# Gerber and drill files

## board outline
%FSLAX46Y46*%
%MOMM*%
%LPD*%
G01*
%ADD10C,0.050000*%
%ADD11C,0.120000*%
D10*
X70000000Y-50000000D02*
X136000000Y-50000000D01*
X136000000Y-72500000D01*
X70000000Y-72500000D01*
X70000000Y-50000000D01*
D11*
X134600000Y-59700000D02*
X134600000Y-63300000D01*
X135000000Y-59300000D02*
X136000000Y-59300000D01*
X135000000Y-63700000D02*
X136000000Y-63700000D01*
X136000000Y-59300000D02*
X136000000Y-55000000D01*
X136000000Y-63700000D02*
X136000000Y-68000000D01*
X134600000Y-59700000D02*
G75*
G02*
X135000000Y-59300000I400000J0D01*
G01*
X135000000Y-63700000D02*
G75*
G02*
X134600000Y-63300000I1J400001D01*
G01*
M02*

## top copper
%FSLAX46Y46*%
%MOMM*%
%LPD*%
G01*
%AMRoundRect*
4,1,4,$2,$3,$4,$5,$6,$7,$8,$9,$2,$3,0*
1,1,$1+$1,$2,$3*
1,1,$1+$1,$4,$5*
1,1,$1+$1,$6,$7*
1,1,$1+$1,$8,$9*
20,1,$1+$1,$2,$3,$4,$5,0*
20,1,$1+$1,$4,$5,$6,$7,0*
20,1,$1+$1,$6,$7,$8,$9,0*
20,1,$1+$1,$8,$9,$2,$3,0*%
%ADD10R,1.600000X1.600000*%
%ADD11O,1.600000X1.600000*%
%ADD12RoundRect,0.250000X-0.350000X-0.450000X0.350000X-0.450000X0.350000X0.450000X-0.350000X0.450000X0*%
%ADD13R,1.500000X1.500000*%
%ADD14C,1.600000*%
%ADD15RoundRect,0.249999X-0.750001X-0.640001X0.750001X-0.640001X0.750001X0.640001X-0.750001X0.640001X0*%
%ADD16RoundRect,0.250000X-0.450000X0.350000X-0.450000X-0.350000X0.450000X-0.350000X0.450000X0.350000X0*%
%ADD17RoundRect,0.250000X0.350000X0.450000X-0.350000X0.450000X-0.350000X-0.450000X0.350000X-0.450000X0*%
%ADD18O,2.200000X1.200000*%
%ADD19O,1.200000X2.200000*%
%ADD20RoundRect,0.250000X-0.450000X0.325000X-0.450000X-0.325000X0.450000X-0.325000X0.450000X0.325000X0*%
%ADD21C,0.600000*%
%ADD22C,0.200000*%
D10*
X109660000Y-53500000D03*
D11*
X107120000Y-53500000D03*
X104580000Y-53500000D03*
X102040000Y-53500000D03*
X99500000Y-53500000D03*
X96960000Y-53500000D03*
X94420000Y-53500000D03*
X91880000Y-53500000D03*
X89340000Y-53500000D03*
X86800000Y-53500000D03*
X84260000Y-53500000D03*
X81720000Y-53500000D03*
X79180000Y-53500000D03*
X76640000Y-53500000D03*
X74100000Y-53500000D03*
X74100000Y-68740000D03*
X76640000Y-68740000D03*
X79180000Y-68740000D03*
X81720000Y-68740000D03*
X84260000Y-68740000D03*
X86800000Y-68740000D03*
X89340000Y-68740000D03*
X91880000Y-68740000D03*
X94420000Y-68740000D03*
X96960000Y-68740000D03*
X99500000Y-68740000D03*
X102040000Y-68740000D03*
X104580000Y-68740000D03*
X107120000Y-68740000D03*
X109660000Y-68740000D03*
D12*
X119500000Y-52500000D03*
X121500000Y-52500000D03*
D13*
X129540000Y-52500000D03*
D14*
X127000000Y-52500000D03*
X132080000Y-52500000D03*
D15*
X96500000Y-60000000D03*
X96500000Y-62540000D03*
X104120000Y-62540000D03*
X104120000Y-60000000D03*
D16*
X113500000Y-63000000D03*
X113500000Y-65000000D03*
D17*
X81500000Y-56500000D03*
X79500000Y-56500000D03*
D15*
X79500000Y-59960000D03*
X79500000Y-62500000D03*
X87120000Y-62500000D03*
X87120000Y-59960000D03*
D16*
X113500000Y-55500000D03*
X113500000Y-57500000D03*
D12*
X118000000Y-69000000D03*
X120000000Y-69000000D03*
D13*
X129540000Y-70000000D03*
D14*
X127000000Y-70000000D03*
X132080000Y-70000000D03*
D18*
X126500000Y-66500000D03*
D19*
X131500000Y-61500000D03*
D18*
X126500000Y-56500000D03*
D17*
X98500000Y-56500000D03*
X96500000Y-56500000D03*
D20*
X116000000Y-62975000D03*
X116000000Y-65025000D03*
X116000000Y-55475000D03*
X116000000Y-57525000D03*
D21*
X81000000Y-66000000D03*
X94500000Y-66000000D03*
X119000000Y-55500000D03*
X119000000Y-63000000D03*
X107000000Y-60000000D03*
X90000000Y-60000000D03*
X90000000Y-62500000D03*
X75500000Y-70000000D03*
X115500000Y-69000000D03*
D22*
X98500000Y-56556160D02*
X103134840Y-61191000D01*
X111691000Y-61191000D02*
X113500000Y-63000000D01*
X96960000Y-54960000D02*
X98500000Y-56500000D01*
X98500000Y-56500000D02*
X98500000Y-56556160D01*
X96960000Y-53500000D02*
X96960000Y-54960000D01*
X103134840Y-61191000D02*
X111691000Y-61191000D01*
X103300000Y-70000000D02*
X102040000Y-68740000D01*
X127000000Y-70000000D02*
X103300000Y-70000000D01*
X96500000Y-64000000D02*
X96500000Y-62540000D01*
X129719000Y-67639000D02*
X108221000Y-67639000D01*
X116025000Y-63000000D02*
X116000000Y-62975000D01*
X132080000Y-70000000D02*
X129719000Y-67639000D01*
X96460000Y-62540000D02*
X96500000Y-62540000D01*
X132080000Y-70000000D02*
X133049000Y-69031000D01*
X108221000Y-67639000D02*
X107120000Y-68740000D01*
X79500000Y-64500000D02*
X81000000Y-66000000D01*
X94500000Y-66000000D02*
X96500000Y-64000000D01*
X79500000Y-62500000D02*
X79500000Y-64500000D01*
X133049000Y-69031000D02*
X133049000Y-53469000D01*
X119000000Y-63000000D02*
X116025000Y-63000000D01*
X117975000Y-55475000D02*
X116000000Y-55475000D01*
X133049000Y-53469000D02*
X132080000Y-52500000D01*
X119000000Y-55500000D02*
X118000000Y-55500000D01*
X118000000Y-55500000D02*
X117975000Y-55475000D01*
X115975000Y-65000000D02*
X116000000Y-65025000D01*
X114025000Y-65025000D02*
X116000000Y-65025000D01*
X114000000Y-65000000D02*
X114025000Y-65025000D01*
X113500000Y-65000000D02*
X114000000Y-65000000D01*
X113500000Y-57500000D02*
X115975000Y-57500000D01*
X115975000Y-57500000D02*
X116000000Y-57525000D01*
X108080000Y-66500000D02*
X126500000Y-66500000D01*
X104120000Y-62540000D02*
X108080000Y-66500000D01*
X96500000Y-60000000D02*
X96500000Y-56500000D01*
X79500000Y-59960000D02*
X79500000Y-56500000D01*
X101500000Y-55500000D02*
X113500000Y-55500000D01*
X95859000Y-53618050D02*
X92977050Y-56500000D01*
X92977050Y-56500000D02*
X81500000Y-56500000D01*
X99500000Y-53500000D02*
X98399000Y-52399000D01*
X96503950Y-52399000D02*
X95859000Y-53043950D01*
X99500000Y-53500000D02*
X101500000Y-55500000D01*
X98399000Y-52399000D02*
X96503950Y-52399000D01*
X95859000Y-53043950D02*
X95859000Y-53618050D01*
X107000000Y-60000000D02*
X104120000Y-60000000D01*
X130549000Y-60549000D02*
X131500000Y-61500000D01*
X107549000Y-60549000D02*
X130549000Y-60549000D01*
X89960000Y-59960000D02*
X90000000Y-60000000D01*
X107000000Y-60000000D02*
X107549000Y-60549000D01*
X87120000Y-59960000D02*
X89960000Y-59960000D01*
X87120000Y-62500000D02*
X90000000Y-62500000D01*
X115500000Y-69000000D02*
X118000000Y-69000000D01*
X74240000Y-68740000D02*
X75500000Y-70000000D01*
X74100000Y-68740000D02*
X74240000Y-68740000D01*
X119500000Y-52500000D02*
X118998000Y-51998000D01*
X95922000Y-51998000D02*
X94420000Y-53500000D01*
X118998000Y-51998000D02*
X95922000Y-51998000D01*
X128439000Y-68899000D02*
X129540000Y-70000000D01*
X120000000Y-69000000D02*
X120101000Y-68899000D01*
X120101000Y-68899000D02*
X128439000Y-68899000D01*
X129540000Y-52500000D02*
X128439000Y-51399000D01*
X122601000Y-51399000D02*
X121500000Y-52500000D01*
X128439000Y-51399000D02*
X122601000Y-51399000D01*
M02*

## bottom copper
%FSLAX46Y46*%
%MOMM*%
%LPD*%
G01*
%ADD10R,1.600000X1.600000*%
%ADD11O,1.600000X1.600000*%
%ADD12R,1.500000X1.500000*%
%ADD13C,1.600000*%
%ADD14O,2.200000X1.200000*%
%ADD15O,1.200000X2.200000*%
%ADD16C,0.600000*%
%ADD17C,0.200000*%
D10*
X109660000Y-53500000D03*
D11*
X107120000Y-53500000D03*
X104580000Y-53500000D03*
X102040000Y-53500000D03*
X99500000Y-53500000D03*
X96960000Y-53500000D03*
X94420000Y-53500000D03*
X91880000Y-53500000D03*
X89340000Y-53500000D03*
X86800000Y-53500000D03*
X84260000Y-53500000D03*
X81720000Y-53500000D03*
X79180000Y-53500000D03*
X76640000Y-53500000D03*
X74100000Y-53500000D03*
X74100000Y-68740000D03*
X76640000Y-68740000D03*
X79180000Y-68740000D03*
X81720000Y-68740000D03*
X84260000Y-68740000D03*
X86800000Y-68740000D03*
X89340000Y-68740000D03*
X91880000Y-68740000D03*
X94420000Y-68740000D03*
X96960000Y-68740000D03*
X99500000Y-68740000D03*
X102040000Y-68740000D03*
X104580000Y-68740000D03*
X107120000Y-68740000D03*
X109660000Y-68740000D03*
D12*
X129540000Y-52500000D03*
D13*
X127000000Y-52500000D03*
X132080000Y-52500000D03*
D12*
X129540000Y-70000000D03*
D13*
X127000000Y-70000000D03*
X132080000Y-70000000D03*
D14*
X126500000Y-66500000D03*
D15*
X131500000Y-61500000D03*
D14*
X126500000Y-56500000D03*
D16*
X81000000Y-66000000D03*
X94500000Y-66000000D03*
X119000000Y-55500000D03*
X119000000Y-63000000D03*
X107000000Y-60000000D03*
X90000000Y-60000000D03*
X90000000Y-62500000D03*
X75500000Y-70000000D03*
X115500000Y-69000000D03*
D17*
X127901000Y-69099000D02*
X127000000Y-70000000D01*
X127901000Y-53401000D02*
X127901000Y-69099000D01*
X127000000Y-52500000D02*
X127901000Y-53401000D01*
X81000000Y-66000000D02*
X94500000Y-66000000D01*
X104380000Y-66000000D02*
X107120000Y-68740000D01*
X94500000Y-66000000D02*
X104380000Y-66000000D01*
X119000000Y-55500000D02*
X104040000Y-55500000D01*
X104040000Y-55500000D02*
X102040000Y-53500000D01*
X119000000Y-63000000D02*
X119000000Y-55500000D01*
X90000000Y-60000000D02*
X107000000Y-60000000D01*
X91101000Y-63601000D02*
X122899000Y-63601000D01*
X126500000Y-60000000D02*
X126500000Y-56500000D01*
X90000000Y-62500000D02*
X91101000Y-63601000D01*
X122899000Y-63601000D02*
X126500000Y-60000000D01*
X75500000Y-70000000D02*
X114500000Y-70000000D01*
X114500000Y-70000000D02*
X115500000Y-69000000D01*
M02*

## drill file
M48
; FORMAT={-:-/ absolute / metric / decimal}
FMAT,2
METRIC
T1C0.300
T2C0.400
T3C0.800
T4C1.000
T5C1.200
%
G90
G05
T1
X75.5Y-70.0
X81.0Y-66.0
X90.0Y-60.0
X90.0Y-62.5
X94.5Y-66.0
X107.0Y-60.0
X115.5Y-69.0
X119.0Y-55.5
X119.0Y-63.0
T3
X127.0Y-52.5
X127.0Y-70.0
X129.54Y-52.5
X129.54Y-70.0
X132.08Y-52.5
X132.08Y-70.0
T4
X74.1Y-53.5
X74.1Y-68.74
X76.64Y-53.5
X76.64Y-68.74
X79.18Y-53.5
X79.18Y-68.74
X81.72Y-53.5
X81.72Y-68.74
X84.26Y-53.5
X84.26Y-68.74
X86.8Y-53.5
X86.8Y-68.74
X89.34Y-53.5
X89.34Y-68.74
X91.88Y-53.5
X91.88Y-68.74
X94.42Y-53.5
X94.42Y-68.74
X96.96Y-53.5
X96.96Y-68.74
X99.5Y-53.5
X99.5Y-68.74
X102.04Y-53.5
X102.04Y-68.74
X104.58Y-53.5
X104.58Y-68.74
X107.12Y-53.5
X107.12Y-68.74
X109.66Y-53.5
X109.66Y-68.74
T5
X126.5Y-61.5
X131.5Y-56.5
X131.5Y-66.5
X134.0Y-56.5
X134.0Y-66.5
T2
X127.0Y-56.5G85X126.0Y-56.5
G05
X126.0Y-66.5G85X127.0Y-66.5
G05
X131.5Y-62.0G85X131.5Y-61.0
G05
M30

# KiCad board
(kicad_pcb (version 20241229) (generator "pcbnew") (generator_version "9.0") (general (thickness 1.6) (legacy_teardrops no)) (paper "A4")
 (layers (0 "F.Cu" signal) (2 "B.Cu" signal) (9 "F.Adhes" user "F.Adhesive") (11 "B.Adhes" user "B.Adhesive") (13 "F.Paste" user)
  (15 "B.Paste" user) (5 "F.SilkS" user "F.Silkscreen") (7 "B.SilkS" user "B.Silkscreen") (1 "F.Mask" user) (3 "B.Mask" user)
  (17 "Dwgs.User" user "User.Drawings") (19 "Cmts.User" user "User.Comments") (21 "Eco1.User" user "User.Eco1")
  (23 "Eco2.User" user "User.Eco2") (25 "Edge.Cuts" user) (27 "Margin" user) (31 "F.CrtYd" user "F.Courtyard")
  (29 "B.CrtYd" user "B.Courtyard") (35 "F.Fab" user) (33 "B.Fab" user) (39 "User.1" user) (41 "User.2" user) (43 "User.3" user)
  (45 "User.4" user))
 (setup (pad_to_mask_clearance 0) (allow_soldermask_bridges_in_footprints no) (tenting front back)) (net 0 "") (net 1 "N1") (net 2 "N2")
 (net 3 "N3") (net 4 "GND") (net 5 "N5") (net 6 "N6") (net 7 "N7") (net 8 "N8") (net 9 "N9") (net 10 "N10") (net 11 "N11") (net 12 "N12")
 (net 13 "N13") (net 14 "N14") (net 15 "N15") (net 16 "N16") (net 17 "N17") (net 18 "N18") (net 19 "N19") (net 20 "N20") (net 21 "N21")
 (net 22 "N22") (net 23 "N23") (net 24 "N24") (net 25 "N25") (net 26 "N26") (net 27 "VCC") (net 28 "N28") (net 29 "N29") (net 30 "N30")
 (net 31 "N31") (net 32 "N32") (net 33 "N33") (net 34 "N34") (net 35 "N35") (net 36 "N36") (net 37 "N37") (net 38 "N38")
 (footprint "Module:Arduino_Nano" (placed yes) (layer "F.Cu") (at 109.66 53.5 -90)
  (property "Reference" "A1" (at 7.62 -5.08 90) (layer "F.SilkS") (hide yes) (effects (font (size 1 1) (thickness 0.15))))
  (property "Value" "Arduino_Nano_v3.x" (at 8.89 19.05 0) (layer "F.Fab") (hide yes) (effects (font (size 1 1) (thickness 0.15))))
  (pad "1" thru_hole rect (at 0 0 270) (size 1.6 1.6) (drill 1) (layers "*.Cu" "*.Mask") (remove_unused_layers no) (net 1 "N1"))
  (pad "2" thru_hole oval (at 0 2.54 270) (size 1.6 1.6) (drill 1) (layers "*.Cu" "*.Mask") (remove_unused_layers no) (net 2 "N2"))
  (pad "3" thru_hole oval (at 0 5.08 270) (size 1.6 1.6) (drill 1) (layers "*.Cu" "*.Mask") (remove_unused_layers no) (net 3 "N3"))
  (pad "4" thru_hole oval (at 0 7.62 270) (size 1.6 1.6) (drill 1) (layers "*.Cu" "*.Mask") (remove_unused_layers no) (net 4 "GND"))
  (pad "5" thru_hole oval (at 0 10.16 270) (size 1.6 1.6) (drill 1) (layers "*.Cu" "*.Mask") (remove_unused_layers no) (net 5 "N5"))
  (pad "6" thru_hole oval (at 0 12.7 270) (size 1.6 1.6) (drill 1) (layers "*.Cu" "*.Mask") (remove_unused_layers no) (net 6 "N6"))
  (pad "7" thru_hole oval (at 0 15.24 270) (size 1.6 1.6) (drill 1) (layers "*.Cu" "*.Mask") (remove_unused_layers no) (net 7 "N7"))
  (pad "8" thru_hole oval (at 0 17.78 270) (size 1.6 1.6) (drill 1) (layers "*.Cu" "*.Mask") (remove_unused_layers no) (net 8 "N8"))
  (pad "9" thru_hole oval (at 0 20.32 270) (size 1.6 1.6) (drill 1) (layers "*.Cu" "*.Mask") (remove_unused_layers no) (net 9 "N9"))
  (pad "10" thru_hole oval (at 0 22.86 270) (size 1.6 1.6) (drill 1) (layers "*.Cu" "*.Mask") (remove_unused_layers no) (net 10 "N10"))
  (pad "11" thru_hole oval (at 0 25.4 270) (size 1.6 1.6) (drill 1) (layers "*.Cu" "*.Mask") (remove_unused_layers no) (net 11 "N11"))
  (pad "12" thru_hole oval (at 0 27.94 270) (size 1.6 1.6) (drill 1) (layers "*.Cu" "*.Mask") (remove_unused_layers no) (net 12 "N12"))
  (pad "13" thru_hole oval (at 0 30.48 270) (size 1.6 1.6) (drill 1) (layers "*.Cu" "*.Mask") (remove_unused_layers no) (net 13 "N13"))
  (pad "14" thru_hole oval (at 0 33.02 270) (size 1.6 1.6) (drill 1) (layers "*.Cu" "*.Mask") (remove_unused_layers no) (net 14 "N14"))
  (pad "15" thru_hole oval (at 0 35.56 270) (size 1.6 1.6) (drill 1) (layers "*.Cu" "*.Mask") (remove_unused_layers no) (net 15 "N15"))
  (pad "16" thru_hole oval (at 15.24 35.56 270) (size 1.6 1.6) (drill 1) (layers "*.Cu" "*.Mask") (remove_unused_layers no) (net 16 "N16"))
  (pad "17" thru_hole oval (at 15.24 33.02 270) (size 1.6 1.6) (drill 1) (layers "*.Cu" "*.Mask") (remove_unused_layers no) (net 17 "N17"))
  (pad "18" thru_hole oval (at 15.24 30.48 270) (size 1.6 1.6) (drill 1) (layers "*.Cu" "*.Mask") (remove_unused_layers no) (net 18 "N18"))
  (pad "19" thru_hole oval (at 15.24 27.94 270) (size 1.6 1.6) (drill 1) (layers "*.Cu" "*.Mask") (remove_unused_layers no) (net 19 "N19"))
  (pad "20" thru_hole oval (at 15.24 25.4 270) (size 1.6 1.6) (drill 1) (layers "*.Cu" "*.Mask") (remove_unused_layers no) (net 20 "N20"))
  (pad "21" thru_hole oval (at 15.24 22.86 270) (size 1.6 1.6) (drill 1) (layers "*.Cu" "*.Mask") (remove_unused_layers no) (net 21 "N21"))
  (pad "22" thru_hole oval (at 15.24 20.32 270) (size 1.6 1.6) (drill 1) (layers "*.Cu" "*.Mask") (remove_unused_layers no) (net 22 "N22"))
  (pad "23" thru_hole oval (at 15.24 17.78 270) (size 1.6 1.6) (drill 1) (layers "*.Cu" "*.Mask") (remove_unused_layers no) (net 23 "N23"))
  (pad "24" thru_hole oval (at 15.24 15.24 270) (size 1.6 1.6) (drill 1) (layers "*.Cu" "*.Mask") (remove_unused_layers no) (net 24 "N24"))
  (pad "25" thru_hole oval (at 15.24 12.7 270) (size 1.6 1.6) (drill 1) (layers "*.Cu" "*.Mask") (remove_unused_layers no) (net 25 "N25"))
  (pad "26" thru_hole oval (at 15.24 10.16 270) (size 1.6 1.6) (drill 1) (layers "*.Cu" "*.Mask") (remove_unused_layers no) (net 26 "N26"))
  (pad "27" thru_hole oval (at 15.24 7.62 270) (size 1.6 1.6) (drill 1) (layers "*.Cu" "*.Mask") (remove_unused_layers no) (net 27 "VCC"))
  (pad "28" thru_hole oval (at 15.24 5.08 270) (size 1.6 1.6) (drill 1) (layers "*.Cu" "*.Mask") (remove_unused_layers no) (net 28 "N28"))
  (pad "29" thru_hole oval (at 15.24 2.54 270) (size 1.6 1.6) (drill 1) (layers "*.Cu" "*.Mask") (remove_unused_layers no) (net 4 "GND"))
  (pad "30" thru_hole oval (at 15.24 0 270) (size 1.6 1.6) (drill 1) (layers "*.Cu" "*.Mask") (remove_unused_layers no) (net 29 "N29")))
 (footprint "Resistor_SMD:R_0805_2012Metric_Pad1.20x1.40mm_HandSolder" (layer "F.Cu") (at 120.5 52.5)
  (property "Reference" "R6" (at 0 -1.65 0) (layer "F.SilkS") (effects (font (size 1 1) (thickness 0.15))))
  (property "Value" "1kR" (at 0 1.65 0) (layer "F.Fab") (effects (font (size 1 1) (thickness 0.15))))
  (pad "1" smd roundrect (at -1 0) (size 1.2 1.4) (layers "F.Cu" "F.Mask" "F.Paste") (roundrect_rratio 0.208333) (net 7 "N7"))
  (pad "2" smd roundrect (at 1 0) (size 1.2 1.4) (layers "F.Cu" "F.Mask" "F.Paste") (roundrect_rratio 0.208333) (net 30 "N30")))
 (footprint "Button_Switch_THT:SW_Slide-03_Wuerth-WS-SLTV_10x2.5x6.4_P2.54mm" (layer "F.Cu") (at 129.54 52.5)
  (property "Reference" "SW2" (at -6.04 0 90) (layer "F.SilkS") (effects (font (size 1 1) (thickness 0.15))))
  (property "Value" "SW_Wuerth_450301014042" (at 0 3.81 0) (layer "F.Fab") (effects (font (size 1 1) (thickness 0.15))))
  (pad "1" thru_hole rect (at 0 0) (size 1.5 1.5) (drill 0.8) (layers "*.Cu" "*.Mask") (remove_unused_layers no) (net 30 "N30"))
  (pad "2" thru_hole circle (at -2.54 0) (size 1.6 1.6) (drill 0.8) (layers "*.Cu" "*.Mask") (remove_unused_layers no) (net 27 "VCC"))
  (pad "3" thru_hole circle (at 2.54 0) (size 1.6 1.6) (drill 0.8) (layers "*.Cu" "*.Mask") (remove_unused_layers no) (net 4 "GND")))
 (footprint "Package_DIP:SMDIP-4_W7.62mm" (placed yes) (layer "F.Cu") (at 100.31 61.27)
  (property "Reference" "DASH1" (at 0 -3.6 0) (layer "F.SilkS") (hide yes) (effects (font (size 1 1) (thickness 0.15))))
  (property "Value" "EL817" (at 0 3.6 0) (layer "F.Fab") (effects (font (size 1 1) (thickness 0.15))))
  (pad "1" smd roundrect (at -3.81 -1.27) (size 2 1.78) (layers "F.Cu" "F.Mask" "F.Paste") (roundrect_rratio 0.140449) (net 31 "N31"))
  (pad "2" smd roundrect (at -3.81 1.27) (size 2 1.78) (layers "F.Cu" "F.Mask" "F.Paste") (roundrect_rratio 0.140449) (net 4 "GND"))
  (pad "3" smd roundrect (at 3.81 1.27) (size 2 1.78) (layers "F.Cu" "F.Mask" "F.Paste") (roundrect_rratio 0.140449) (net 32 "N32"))
  (pad "4" smd roundrect (at 3.81 -1.27) (size 2 1.78) (layers "F.Cu" "F.Mask" "F.Paste") (roundrect_rratio 0.140449) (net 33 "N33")))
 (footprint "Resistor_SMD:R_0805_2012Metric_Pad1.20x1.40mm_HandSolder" (layer "F.Cu") (at 113.5 64 -90)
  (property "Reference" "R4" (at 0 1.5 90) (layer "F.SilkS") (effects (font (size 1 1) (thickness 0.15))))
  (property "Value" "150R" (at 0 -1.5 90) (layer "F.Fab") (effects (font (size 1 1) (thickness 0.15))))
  (pad "1" smd roundrect (at -1 0 270) (size 1.2 1.4) (layers "F.Cu" "F.Mask" "F.Paste") (roundrect_rratio 0.208333) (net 6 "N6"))
  (pad "2" smd roundrect (at 1 0 270) (size 1.2 1.4) (layers "F.Cu" "F.Mask" "F.Paste") (roundrect_rratio 0.208333) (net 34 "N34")))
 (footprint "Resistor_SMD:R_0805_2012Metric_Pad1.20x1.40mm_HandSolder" (layer "F.Cu") (at 80.5 56.5 180)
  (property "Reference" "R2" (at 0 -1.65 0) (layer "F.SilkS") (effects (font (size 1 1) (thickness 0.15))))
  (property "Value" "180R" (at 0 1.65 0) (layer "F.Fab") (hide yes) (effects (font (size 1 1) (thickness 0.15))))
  (pad "1" smd roundrect (at -1 0 180) (size 1.2 1.4) (layers "F.Cu" "F.Mask" "F.Paste") (roundrect_rratio 0.208333) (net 5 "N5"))
  (pad "2" smd roundrect (at 1 0 180) (size 1.2 1.4) (layers "F.Cu" "F.Mask" "F.Paste") (roundrect_rratio 0.208333) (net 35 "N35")))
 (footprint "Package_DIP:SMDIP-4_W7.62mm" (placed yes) (layer "F.Cu") (at 83.31 61.23)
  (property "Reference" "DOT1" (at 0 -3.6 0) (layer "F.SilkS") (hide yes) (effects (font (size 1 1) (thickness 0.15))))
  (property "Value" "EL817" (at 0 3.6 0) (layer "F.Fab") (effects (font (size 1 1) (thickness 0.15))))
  (pad "1" smd roundrect (at -3.81 -1.27) (size 2 1.78) (layers "F.Cu" "F.Mask" "F.Paste") (roundrect_rratio 0.140449) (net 35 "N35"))
  (pad "2" smd roundrect (at -3.81 1.27) (size 2 1.78) (layers "F.Cu" "F.Mask" "F.Paste") (roundrect_rratio 0.140449) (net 4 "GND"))
  (pad "3" smd roundrect (at 3.81 1.27) (size 2 1.78) (layers "F.Cu" "F.Mask" "F.Paste") (roundrect_rratio 0.140449) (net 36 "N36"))
  (pad "4" smd roundrect (at 3.81 -1.27) (size 2 1.78) (layers "F.Cu" "F.Mask" "F.Paste") (roundrect_rratio 0.140449) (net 33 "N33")))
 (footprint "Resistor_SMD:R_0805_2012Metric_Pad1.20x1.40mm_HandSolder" (layer "F.Cu") (at 113.5 56.5 -90)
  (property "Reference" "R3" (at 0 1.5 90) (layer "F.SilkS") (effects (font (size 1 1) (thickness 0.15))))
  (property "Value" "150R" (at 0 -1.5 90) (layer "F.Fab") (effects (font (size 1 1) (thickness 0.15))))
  (pad "1" smd roundrect (at -1 0 270) (size 1.2 1.4) (layers "F.Cu" "F.Mask" "F.Paste") (roundrect_rratio 0.208333) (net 5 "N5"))
  (pad "2" smd roundrect (at 1 0 270) (size 1.2 1.4) (layers "F.Cu" "F.Mask" "F.Paste") (roundrect_rratio 0.208333) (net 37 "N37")))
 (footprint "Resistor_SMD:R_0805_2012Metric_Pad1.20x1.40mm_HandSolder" (layer "F.Cu") (at 119 69)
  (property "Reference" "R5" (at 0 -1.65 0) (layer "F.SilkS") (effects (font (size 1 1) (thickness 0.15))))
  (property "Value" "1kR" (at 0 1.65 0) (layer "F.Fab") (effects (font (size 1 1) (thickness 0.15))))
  (pad "1" smd roundrect (at -1 0) (size 1.2 1.4) (layers "F.Cu" "F.Mask" "F.Paste") (roundrect_rratio 0.208333) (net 16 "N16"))
  (pad "2" smd roundrect (at 1 0) (size 1.2 1.4) (layers "F.Cu" "F.Mask" "F.Paste") (roundrect_rratio 0.208333) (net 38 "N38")))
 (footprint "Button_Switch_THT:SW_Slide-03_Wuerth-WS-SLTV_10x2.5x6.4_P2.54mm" (layer "F.Cu") (at 129.54 70)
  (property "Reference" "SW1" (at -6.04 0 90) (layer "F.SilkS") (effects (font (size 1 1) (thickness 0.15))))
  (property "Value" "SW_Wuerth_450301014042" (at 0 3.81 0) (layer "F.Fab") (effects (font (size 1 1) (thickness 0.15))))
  (pad "1" thru_hole rect (at 0 0) (size 1.5 1.5) (drill 0.8) (layers "*.Cu" "*.Mask") (remove_unused_layers no) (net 38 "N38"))
  (pad "2" thru_hole circle (at -2.54 0) (size 1.6 1.6) (drill 0.8) (layers "*.Cu" "*.Mask") (remove_unused_layers no) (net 27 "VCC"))
  (pad "3" thru_hole circle (at 2.54 0) (size 1.6 1.6) (drill 0.8) (layers "*.Cu" "*.Mask") (remove_unused_layers no) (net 4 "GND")))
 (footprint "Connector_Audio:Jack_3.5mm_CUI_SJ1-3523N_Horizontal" (layer "F.Cu") (at 131.5 61.5 90)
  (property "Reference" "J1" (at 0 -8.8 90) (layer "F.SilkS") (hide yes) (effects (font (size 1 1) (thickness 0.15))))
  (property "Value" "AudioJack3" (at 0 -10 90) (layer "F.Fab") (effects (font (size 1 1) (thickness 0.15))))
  (fp_line (start 1.8 3.1) (end -1.8 3.1) (stroke (width 0.12) (type solid)) (layer "Edge.Cuts"))
  (fp_line (start 2.2 3.5) (end 2.2 4.5) (stroke (width 0.12) (type solid)) (layer "Edge.Cuts"))
  (fp_line (start -2.2 3.5) (end -2.2 4.5) (stroke (width 0.12) (type solid)) (layer "Edge.Cuts"))
  (fp_line (start 2.2 4.5) (end 6.5 4.5) (stroke (width 0.12) (type solid)) (layer "Edge.Cuts"))
  (fp_line (start -2.2 4.5) (end -6.5 4.5) (stroke (width 0.12) (type solid)) (layer "Edge.Cuts"))
  (fp_arc (start 1.8 3.1) (mid 2.082843 3.217157) (end 2.2 3.5) (stroke (width 0.12) (type solid)) (layer "Edge.Cuts"))
  (fp_arc (start -2.2 3.5) (mid -2.082843 3.217158) (end -1.8 3.1) (stroke (width 0.12) (type solid)) (layer "Edge.Cuts"))
  (pad "" np_thru_hole circle (at -5 0 90) (size 1.2 1.2) (drill 1.2) (layers "*.Cu" "*.Mask"))
  (pad "" np_thru_hole circle (at -5 2.5 90) (size 1.2 1.2) (drill 1.2) (layers "*.Cu" "*.Mask"))
  (pad "" np_thru_hole circle (at 0 -5 90) (size 1.2 1.2) (drill 1.2) (layers "*.Cu" "*.Mask"))
  (pad "" np_thru_hole circle (at 5 0 90) (size 1.2 1.2) (drill 1.2) (layers "*.Cu" "*.Mask"))
  (pad "" np_thru_hole circle (at 5 2.5 90) (size 1.2 1.2) (drill 1.2) (layers "*.Cu" "*.Mask"))
  (pad "R" thru_hole oval (at -5 -5 90) (size 1.2 2.2) (drill oval 0.4 1.4) (layers "*.Cu" "*.Mask") (remove_unused_layers no)
   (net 32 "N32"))
  (pad "S" thru_hole oval (at 0 0 90) (size 2.2 1.2) (drill oval 1.4 0.4) (layers "*.Cu" "*.Mask") (remove_unused_layers no) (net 33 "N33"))
  (pad "T" thru_hole oval (at 5 -5 270) (size 1.2 2.2) (drill oval 0.4 1.4) (layers "*.Cu" "*.Mask") (remove_unused_layers no)
   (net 36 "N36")))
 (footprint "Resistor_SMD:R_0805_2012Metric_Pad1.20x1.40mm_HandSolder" (layer "F.Cu") (at 97.5 56.5 180)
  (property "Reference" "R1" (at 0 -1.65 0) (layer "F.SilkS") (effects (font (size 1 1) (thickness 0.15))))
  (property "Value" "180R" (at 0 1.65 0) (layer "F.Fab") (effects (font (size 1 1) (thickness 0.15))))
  (pad "1" smd roundrect (at -1 0 180) (size 1.2 1.4) (layers "F.Cu" "F.Mask" "F.Paste") (roundrect_rratio 0.208333) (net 6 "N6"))
  (pad "2" smd roundrect (at 1 0 180) (size 1.2 1.4) (layers "F.Cu" "F.Mask" "F.Paste") (roundrect_rratio 0.208333) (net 31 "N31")))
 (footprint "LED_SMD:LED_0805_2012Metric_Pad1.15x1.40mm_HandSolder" (layer "F.Cu") (at 116 64 -90)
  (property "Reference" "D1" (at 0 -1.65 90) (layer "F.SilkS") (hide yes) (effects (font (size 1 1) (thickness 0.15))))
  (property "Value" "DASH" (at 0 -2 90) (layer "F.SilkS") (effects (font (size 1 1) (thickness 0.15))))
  (pad "1" smd roundrect (at -1.025 0 270) (size 1.15 1.4) (layers "F.Cu" "F.Mask" "F.Paste") (roundrect_rratio 0.217391) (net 4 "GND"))
  (pad "2" smd roundrect (at 1.025 0 270) (size 1.15 1.4) (layers "F.Cu" "F.Mask" "F.Paste") (roundrect_rratio 0.217391) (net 34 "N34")))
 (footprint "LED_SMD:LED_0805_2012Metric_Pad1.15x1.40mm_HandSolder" (layer "F.Cu") (at 116 56.5 -90)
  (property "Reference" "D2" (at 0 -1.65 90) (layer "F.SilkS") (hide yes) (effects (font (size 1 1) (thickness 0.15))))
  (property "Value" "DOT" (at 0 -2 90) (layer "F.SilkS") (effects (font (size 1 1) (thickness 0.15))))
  (pad "1" smd roundrect (at -1.025 0 270) (size 1.15 1.4) (layers "F.Cu" "F.Mask" "F.Paste") (roundrect_rratio 0.217391) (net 4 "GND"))
  (pad "2" smd roundrect (at 1.025 0 270) (size 1.15 1.4) (layers "F.Cu" "F.Mask" "F.Paste") (roundrect_rratio 0.217391) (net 37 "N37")))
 (gr_rect (start 70 50) (end 136 72.5) (stroke (width 0.05) (type default)) (fill no) (layer "Edge.Cuts"))
 (segment (start 98.5 56.55616) (end 103.13484 61.191) (width 0.2) (layer "F.Cu") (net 6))
 (segment (start 111.691 61.191) (end 113.5 63) (width 0.2) (layer "F.Cu") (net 6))
 (segment (start 96.96 54.96) (end 98.5 56.5) (width 0.2) (layer "F.Cu") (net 6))
 (segment (start 98.5 56.5) (end 98.5 56.55616) (width 0.2) (layer "F.Cu") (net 6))
 (segment (start 96.96 53.5) (end 96.96 54.96) (width 0.2) (layer "F.Cu") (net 6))
 (segment (start 103.13484 61.191) (end 111.691 61.191) (width 0.2) (layer "F.Cu") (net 6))
 (segment (start 103.3 70) (end 102.04 68.74) (width 0.2) (layer "F.Cu") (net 27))
 (segment (start 127 70) (end 103.3 70) (width 0.2) (layer "F.Cu") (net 27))
 (segment (start 127.901 69.099) (end 127 70) (width 0.2) (layer "B.Cu") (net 27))
 (segment (start 127.901 53.401) (end 127.901 69.099) (width 0.2) (layer "B.Cu") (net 27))
 (segment (start 127 52.5) (end 127.901 53.401) (width 0.2) (layer "B.Cu") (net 27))
 (segment (start 96.5 64) (end 96.5 62.54) (width 0.2) (layer "F.Cu") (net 4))
 (segment (start 129.719 67.639) (end 108.221 67.639) (width 0.2) (layer "F.Cu") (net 4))
 (segment (start 116.025 63) (end 116 62.975) (width 0.2) (layer "F.Cu") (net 4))
 (segment (start 132.08 70) (end 129.719 67.639) (width 0.2) (layer "F.Cu") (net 4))
 (segment (start 96.46 62.54) (end 96.5 62.54) (width 0.2) (layer "F.Cu") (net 4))
 (segment (start 132.08 70) (end 133.049 69.031) (width 0.2) (layer "F.Cu") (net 4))
 (segment (start 108.221 67.639) (end 107.12 68.74) (width 0.2) (layer "F.Cu") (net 4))
 (segment (start 79.5 64.5) (end 81 66) (width 0.2) (layer "F.Cu") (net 4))
 (segment (start 94.5 66) (end 96.5 64) (width 0.2) (layer "F.Cu") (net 4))
 (segment (start 79.5 62.5) (end 79.5 64.5) (width 0.2) (layer "F.Cu") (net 4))
 (segment (start 133.049 69.031) (end 133.049 53.469) (width 0.2) (layer "F.Cu") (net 4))
 (segment (start 119 63) (end 116.025 63) (width 0.2) (layer "F.Cu") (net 4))
 (segment (start 117.975 55.475) (end 116 55.475) (width 0.2) (layer "F.Cu") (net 4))
 (segment (start 133.049 53.469) (end 132.08 52.5) (width 0.2) (layer "F.Cu") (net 4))
 (segment (start 119 55.5) (end 118 55.5) (width 0.2) (layer "F.Cu") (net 4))
 (segment (start 118 55.5) (end 117.975 55.475) (width 0.2) (layer "F.Cu") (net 4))
 (via (at 81 66) (size 0.6) (drill 0.3) (layers "F.Cu" "B.Cu") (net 4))
 (via (at 94.5 66) (size 0.6) (drill 0.3) (layers "F.Cu" "B.Cu") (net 4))
 (via (at 119 55.5) (size 0.6) (drill 0.3) (layers "F.Cu" "B.Cu") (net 4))
 (via (at 119 63) (size 0.6) (drill 0.3) (layers "F.Cu" "B.Cu") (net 4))
 (segment (start 81 66) (end 94.5 66) (width 0.2) (layer "B.Cu") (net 4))
 (segment (start 104.38 66) (end 107.12 68.74) (width 0.2) (layer "B.Cu") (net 4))
 (segment (start 94.5 66) (end 104.38 66) (width 0.2) (layer "B.Cu") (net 4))
 (segment (start 119 55.5) (end 104.04 55.5) (width 0.2) (layer "B.Cu") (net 4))
 (segment (start 104.04 55.5) (end 102.04 53.5) (width 0.2) (layer "B.Cu") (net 4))
 (segment (start 119 63) (end 119 55.5) (width 0.2) (layer "B.Cu") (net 4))
 (segment (start 115.975 65) (end 116 65.025) (width 0.2) (layer "F.Cu") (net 34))
 (segment (start 114.025 65.025) (end 116 65.025) (width 0.2) (layer "F.Cu") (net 34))
 (segment (start 114 65) (end 114.025 65.025) (width 0.2) (layer "F.Cu") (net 34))
 (segment (start 113.5 65) (end 114 65) (width 0.2) (layer "F.Cu") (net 34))
 (segment (start 113.5 57.5) (end 115.975 57.5) (width 0.2) (layer "F.Cu") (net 37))
 (segment (start 115.975 57.5) (end 116 57.525) (width 0.2) (layer "F.Cu") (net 37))
 (segment (start 108.08 66.5) (end 126.5 66.5) (width 0.2) (layer "F.Cu") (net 32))
 (segment (start 104.12 62.54) (end 108.08 66.5) (width 0.2) (layer "F.Cu") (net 32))
 (segment (start 96.5 60) (end 96.5 56.5) (width 0.2) (layer "F.Cu") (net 31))
 (segment (start 79.5 59.96) (end 79.5 56.5) (width 0.2) (layer "F.Cu") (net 35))
 (segment (start 101.5 55.5) (end 113.5 55.5) (width 0.2) (layer "F.Cu") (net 5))
 (segment (start 95.859 53.61805) (end 92.97705 56.5) (width 0.2) (layer "F.Cu") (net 5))
 (segment (start 92.97705 56.5) (end 81.5 56.5) (width 0.2) (layer "F.Cu") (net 5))
 (segment (start 99.5 53.5) (end 98.399 52.399) (width 0.2) (layer "F.Cu") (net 5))
 (segment (start 96.50395 52.399) (end 95.859 53.04395) (width 0.2) (layer "F.Cu") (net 5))
 (segment (start 99.5 53.5) (end 101.5 55.5) (width 0.2) (layer "F.Cu") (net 5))
 (segment (start 98.399 52.399) (end 96.50395 52.399) (width 0.2) (layer "F.Cu") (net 5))
 (segment (start 95.859 53.04395) (end 95.859 53.61805) (width 0.2) (layer "F.Cu") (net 5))
 (segment (start 107 60) (end 104.12 60) (width 0.2) (layer "F.Cu") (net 33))
 (segment (start 130.549 60.549) (end 131.5 61.5) (width 0.2) (layer "F.Cu") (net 33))
 (segment (start 107.549 60.549) (end 130.549 60.549) (width 0.2) (layer "F.Cu") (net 33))
 (segment (start 89.96 59.96) (end 90 60) (width 0.2) (layer "F.Cu") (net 33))
 (segment (start 107 60) (end 107.549 60.549) (width 0.2) (layer "F.Cu") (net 33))
 (segment (start 87.12 59.96) (end 89.96 59.96) (width 0.2) (layer "F.Cu") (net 33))
 (via (at 107 60) (size 0.6) (drill 0.3) (layers "F.Cu" "B.Cu") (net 33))
 (via (at 90 60) (size 0.6) (drill 0.3) (layers "F.Cu" "B.Cu") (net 33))
 (segment (start 90 60) (end 107 60) (width 0.2) (layer "B.Cu") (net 33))
 (segment (start 87.12 62.5) (end 90 62.5) (width 0.2) (layer "F.Cu") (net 36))
 (via (at 90 62.5) (size 0.6) (drill 0.3) (layers "F.Cu" "B.Cu") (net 36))
 (segment (start 91.101 63.601) (end 122.899 63.601) (width 0.2) (layer "B.Cu") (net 36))
 (segment (start 126.5 60) (end 126.5 56.5) (width 0.2) (layer "B.Cu") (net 36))
 (segment (start 90 62.5) (end 91.101 63.601) (width 0.2) (layer "B.Cu") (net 36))
 (segment (start 122.899 63.601) (end 126.5 60) (width 0.2) (layer "B.Cu") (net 36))
 (segment (start 115.5 69) (end 118 69) (width 0.2) (layer "F.Cu") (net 16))
 (segment (start 74.24 68.74) (end 75.5 70) (width 0.2) (layer "F.Cu") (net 16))
 (segment (start 74.1 68.74) (end 74.24 68.74) (width 0.2) (layer "F.Cu") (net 16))
 (via (at 75.5 70) (size 0.6) (drill 0.3) (layers "F.Cu" "B.Cu") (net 16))
 (via (at 115.5 69) (size 0.6) (drill 0.3) (layers "F.Cu" "B.Cu") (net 16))
 (segment (start 75.5 70) (end 114.5 70) (width 0.2) (layer "B.Cu") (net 16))
 (segment (start 114.5 70) (end 115.5 69) (width 0.2) (layer "B.Cu") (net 16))
 (segment (start 119.5 52.5) (end 118.998 51.998) (width 0.2) (layer "F.Cu") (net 7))
 (segment (start 95.922 51.998) (end 94.42 53.5) (width 0.2) (layer "F.Cu") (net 7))
 (segment (start 118.998 51.998) (end 95.922 51.998) (width 0.2) (layer "F.Cu") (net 7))
 (segment (start 128.439 68.899) (end 129.54 70) (width 0.2) (layer "F.Cu") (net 38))
 (segment (start 120 69) (end 120.101 68.899) (width 0.2) (layer "F.Cu") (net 38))
 (segment (start 120.101 68.899) (end 128.439 68.899) (width 0.2) (layer "F.Cu") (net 38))
 (segment (start 129.54 52.5) (end 128.439 51.399) (width 0.2) (layer "F.Cu") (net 30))
 (segment (start 122.601 51.399) (end 121.5 52.5) (width 0.2) (layer "F.Cu") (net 30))
 (segment (start 128.439 51.399) (end 122.601 51.399) (width 0.2) (layer "F.Cu") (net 30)))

